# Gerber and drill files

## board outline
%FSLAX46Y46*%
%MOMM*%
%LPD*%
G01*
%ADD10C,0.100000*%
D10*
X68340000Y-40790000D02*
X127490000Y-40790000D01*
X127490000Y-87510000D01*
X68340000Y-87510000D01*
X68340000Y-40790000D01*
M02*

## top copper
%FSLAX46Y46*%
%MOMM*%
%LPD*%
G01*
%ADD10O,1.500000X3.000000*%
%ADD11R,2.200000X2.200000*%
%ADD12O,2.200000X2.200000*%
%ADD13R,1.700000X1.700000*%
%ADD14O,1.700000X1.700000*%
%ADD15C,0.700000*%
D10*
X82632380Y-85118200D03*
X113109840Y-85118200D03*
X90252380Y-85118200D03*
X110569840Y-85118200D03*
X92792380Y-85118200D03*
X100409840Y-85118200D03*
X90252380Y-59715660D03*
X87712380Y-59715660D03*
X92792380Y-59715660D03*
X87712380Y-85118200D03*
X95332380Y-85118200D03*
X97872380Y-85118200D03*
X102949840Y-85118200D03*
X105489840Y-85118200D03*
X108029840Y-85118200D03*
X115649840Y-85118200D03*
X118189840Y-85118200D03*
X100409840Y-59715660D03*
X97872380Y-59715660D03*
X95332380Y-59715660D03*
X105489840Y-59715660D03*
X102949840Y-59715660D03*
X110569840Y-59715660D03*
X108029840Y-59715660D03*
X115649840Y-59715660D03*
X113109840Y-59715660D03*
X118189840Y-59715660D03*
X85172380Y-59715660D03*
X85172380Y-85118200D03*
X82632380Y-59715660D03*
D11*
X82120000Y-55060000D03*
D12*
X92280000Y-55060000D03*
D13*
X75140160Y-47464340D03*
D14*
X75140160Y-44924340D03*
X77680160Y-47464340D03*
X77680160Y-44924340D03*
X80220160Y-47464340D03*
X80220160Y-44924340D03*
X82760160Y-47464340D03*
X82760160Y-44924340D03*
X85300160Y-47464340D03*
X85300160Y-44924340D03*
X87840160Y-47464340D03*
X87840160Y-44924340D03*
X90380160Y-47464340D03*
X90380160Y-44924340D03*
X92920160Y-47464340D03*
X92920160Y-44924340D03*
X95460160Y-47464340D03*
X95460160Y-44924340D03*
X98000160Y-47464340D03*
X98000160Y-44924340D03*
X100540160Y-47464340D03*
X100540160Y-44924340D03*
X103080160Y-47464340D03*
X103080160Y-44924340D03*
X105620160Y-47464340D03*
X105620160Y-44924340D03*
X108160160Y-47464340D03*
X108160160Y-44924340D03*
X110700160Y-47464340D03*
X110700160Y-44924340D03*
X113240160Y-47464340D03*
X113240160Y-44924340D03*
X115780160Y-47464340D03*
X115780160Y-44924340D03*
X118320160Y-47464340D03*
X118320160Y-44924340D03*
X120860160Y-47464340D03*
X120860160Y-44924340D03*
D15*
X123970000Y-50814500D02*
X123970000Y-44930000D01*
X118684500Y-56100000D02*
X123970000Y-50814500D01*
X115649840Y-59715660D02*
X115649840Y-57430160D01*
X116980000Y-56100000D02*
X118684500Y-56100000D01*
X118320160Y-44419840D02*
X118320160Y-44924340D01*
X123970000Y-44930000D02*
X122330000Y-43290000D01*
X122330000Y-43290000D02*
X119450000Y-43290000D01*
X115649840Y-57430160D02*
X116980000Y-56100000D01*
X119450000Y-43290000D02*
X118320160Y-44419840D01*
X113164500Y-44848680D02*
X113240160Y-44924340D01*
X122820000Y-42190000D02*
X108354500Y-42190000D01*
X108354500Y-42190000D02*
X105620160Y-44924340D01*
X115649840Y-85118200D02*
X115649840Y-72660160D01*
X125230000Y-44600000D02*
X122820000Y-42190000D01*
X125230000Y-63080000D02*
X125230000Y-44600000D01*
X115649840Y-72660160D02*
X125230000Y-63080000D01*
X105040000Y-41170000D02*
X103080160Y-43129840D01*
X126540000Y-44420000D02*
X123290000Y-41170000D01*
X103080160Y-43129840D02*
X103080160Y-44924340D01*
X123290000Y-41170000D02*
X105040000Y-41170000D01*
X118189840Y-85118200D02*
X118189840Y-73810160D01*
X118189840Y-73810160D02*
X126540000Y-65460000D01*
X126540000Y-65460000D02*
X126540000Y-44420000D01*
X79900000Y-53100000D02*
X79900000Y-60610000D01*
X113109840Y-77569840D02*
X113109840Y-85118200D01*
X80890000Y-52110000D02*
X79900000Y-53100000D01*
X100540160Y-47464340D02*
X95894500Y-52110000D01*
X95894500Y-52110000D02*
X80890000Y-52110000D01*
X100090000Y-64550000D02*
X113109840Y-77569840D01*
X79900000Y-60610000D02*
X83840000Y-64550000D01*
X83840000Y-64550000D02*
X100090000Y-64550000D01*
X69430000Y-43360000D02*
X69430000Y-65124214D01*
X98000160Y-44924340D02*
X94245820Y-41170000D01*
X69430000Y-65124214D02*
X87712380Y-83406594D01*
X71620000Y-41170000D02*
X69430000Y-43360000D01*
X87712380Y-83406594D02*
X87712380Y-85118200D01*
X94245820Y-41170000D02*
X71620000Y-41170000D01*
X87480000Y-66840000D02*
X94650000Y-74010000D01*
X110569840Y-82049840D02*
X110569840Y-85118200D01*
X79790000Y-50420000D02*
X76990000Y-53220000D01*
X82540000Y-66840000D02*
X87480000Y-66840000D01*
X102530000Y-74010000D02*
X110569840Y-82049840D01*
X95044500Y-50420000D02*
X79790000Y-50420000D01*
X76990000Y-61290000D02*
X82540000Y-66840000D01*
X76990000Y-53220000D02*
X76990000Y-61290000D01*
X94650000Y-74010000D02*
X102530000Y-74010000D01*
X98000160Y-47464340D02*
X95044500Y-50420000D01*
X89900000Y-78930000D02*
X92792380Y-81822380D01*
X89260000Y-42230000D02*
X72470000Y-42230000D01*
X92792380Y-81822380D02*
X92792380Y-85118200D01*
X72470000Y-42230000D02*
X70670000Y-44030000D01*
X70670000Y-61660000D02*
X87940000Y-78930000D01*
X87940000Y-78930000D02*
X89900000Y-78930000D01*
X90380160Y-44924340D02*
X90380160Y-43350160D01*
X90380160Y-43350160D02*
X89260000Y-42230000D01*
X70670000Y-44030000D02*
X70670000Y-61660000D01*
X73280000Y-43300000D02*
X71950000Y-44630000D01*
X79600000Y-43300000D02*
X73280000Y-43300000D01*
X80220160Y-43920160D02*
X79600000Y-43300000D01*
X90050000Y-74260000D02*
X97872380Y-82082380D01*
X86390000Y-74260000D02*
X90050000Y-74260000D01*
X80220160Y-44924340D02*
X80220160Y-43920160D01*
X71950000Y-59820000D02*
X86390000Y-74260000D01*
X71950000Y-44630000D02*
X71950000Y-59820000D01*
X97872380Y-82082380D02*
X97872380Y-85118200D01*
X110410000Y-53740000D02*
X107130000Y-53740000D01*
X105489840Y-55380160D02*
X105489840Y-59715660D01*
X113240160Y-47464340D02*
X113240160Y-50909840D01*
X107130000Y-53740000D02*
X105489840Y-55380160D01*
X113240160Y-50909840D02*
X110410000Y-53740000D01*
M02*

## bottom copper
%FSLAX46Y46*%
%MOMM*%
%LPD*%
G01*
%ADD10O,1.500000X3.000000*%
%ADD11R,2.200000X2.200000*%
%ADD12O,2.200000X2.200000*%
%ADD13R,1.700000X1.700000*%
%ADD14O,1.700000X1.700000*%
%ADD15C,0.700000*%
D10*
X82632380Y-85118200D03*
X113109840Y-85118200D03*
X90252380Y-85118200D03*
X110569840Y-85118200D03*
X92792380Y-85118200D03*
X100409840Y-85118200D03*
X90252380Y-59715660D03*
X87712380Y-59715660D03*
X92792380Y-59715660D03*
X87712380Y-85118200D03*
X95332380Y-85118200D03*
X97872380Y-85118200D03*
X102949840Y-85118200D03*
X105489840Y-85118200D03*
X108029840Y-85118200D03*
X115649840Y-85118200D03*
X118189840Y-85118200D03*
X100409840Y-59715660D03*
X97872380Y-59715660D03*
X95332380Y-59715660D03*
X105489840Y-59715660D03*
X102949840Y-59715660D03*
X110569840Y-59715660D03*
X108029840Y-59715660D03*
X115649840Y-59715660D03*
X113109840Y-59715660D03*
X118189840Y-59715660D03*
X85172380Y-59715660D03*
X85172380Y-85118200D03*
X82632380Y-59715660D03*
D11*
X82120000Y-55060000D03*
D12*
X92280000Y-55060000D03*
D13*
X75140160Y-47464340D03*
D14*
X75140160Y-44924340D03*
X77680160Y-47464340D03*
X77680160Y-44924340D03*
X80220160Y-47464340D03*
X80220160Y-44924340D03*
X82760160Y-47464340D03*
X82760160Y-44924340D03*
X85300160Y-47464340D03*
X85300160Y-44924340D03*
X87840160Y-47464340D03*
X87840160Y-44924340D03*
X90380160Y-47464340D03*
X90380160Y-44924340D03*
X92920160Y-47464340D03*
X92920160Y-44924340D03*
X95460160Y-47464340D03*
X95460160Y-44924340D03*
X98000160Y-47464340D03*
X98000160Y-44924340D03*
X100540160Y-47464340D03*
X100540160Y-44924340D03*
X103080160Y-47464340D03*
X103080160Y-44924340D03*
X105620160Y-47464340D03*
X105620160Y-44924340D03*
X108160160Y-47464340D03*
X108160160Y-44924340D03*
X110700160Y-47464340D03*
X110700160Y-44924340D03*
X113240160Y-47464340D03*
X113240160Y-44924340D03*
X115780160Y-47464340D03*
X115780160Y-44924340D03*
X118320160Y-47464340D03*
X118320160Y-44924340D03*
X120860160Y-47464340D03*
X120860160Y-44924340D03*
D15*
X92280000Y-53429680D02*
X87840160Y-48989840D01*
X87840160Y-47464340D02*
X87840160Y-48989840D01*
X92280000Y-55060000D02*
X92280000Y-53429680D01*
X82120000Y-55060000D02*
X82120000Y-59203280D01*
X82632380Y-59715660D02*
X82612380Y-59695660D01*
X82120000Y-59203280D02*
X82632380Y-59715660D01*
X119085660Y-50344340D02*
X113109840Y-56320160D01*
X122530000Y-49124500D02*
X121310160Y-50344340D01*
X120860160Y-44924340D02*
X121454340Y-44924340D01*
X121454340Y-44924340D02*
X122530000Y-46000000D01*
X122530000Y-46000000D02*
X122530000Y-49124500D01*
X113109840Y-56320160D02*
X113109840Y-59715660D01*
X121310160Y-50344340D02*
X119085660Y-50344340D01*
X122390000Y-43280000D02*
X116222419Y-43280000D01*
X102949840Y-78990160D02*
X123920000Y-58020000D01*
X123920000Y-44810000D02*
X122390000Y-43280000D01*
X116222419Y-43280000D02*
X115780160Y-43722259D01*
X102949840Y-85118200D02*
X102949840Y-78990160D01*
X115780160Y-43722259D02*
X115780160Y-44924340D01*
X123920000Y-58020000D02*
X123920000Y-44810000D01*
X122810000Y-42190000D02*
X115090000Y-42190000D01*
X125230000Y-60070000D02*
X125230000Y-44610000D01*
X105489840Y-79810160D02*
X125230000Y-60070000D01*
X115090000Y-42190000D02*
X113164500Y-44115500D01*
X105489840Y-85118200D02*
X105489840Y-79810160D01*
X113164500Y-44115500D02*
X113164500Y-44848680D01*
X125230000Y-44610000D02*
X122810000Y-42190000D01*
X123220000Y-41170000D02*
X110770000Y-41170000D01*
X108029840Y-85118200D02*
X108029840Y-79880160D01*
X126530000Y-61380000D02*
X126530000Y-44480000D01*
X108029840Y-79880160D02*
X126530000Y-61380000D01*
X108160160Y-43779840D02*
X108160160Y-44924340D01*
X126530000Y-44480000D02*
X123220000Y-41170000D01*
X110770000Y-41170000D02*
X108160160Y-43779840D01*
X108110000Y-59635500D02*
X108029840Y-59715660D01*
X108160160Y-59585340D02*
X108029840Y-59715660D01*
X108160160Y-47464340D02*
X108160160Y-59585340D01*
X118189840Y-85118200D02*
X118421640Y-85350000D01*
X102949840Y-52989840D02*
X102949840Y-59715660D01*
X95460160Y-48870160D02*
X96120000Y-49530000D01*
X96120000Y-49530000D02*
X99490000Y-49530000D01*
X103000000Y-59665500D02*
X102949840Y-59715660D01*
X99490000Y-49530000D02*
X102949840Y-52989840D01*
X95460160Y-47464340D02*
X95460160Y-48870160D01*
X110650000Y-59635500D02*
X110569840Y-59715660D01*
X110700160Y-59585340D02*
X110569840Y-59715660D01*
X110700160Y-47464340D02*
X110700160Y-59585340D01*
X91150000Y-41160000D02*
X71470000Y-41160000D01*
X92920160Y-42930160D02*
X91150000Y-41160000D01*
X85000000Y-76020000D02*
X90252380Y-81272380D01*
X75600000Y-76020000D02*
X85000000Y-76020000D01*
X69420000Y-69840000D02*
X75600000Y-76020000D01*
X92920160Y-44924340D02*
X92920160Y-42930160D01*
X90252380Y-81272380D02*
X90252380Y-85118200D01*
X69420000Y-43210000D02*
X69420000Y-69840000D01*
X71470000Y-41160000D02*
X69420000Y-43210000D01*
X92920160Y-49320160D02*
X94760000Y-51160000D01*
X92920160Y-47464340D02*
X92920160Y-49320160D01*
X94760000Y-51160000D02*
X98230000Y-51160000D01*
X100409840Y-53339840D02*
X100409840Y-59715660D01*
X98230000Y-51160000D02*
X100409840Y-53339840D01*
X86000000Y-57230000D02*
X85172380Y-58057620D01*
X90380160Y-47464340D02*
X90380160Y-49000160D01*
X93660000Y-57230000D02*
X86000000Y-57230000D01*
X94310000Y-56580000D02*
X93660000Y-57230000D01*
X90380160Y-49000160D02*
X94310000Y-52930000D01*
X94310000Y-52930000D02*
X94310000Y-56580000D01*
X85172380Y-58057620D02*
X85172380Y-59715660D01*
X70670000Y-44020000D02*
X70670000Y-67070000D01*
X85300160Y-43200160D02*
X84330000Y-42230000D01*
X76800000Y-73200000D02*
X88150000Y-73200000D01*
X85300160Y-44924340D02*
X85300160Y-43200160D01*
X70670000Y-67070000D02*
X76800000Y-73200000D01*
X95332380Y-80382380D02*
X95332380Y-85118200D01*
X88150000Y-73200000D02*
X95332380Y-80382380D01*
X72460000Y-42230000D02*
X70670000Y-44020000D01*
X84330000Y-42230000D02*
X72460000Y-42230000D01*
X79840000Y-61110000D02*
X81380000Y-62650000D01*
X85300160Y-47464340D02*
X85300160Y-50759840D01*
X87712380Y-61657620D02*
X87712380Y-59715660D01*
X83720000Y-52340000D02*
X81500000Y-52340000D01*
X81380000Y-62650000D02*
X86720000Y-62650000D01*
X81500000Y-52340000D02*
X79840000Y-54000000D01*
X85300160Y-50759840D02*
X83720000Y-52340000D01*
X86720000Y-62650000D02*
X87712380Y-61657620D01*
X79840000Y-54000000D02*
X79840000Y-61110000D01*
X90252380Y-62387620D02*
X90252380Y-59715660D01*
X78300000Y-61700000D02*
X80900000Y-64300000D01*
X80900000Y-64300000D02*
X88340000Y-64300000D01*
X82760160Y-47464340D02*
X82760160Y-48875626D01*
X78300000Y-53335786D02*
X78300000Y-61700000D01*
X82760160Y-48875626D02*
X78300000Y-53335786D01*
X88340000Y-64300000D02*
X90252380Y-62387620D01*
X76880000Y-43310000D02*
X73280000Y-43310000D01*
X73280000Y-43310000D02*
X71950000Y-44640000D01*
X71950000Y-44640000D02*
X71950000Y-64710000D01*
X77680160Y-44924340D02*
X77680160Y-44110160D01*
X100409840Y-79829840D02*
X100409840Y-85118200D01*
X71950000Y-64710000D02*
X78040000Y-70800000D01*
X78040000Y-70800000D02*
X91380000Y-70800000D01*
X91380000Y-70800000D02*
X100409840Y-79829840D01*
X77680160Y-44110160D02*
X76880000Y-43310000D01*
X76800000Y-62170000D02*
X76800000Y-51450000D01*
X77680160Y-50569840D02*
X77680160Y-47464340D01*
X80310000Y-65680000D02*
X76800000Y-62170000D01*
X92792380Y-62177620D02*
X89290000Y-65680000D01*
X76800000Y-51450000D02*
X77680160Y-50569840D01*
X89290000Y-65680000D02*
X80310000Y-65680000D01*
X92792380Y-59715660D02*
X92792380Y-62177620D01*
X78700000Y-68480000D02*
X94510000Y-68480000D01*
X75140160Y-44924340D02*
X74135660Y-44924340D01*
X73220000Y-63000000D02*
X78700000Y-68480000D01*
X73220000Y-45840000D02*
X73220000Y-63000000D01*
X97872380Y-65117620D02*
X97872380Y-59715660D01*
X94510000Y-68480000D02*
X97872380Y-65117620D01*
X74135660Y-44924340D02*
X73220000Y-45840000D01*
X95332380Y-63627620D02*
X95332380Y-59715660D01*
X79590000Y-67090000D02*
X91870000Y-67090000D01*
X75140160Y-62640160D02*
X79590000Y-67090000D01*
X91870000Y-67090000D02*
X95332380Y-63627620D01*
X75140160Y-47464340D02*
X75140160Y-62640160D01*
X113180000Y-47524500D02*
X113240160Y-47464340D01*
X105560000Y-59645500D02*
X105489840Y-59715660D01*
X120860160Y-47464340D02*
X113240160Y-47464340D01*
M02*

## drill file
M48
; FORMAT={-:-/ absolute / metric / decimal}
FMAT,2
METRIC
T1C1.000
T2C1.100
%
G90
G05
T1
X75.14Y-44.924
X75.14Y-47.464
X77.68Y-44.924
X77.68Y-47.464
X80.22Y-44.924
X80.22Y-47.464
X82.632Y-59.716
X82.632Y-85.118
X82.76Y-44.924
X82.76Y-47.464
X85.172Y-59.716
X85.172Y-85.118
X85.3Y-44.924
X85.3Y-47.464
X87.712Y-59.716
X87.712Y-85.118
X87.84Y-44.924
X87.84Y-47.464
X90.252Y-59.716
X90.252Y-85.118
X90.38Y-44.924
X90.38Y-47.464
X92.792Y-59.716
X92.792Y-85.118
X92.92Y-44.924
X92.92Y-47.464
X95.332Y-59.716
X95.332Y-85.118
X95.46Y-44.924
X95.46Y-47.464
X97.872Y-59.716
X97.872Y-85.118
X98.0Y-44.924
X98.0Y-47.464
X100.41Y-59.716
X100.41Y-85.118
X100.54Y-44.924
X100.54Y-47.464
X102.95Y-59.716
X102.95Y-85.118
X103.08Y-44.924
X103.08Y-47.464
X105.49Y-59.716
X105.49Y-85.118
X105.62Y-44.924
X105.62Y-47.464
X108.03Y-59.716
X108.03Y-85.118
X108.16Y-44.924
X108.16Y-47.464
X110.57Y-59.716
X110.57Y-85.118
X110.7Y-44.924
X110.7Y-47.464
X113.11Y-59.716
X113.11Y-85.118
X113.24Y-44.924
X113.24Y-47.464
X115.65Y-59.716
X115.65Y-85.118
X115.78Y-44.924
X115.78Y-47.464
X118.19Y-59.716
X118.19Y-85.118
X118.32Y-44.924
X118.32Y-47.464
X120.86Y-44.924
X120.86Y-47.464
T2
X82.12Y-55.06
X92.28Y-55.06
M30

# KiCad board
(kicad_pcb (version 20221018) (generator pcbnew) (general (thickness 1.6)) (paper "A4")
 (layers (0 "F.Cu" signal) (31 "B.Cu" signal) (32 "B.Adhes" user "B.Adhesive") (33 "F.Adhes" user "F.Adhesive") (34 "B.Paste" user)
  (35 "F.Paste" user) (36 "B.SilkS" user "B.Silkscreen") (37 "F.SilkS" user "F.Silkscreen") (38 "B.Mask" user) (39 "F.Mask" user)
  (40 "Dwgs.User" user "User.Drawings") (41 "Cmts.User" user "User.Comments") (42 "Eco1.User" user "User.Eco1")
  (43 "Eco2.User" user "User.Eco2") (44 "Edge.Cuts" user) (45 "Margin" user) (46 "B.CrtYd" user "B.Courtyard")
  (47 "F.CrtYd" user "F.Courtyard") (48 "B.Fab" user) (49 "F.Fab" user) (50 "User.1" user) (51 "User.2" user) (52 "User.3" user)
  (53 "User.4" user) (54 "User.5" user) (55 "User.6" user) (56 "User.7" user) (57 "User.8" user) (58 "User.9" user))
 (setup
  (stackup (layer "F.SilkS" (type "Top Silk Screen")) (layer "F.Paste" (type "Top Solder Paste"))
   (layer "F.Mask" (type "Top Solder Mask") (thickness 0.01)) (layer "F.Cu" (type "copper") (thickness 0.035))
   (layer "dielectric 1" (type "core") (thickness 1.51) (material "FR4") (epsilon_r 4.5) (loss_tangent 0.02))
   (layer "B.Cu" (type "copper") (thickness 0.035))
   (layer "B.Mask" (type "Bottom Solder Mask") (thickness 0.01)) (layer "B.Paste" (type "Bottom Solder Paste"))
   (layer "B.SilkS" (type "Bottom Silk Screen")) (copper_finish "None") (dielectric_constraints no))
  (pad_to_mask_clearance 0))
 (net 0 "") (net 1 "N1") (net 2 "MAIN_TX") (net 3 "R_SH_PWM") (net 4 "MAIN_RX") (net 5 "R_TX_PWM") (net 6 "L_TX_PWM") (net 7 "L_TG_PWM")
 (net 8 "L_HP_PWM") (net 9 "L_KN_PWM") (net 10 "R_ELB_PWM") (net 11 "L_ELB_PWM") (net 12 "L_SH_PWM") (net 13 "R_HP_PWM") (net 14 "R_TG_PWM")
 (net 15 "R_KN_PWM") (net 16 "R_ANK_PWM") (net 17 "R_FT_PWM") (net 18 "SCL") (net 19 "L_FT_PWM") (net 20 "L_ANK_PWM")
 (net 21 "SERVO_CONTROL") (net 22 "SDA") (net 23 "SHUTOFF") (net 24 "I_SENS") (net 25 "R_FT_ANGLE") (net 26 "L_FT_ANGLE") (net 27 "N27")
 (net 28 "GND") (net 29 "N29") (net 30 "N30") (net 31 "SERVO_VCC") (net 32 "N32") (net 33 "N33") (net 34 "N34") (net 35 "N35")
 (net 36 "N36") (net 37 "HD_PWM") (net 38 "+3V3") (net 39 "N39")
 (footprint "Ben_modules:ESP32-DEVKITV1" (layer "F.Cu") (at 99.15 72.85)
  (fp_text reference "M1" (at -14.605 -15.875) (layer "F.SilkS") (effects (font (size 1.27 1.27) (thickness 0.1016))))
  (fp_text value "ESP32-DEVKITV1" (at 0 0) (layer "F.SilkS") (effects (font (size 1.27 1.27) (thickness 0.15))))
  (pad "3V3" thru_hole oval (at -16.51762 12.2682) (size 1.5 3) (drill 1) (layers "*.Cu" "*.Mask") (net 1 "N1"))
  (pad "D1" thru_hole oval (at 13.95984 12.2682) (size 1.5 3) (drill 1) (layers "*.Cu" "*.Mask") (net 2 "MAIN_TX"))
  (pad "D2" thru_hole oval (at -8.89762 12.2682) (size 1.5 3) (drill 1) (layers "*.Cu" "*.Mask") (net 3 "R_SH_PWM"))
  (pad "D3" thru_hole oval (at 11.41984 12.2682) (size 1.5 3) (drill 1) (layers "*.Cu" "*.Mask") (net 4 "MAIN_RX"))
  (pad "D4" thru_hole oval (at -6.35762 12.2682) (size 1.5 3) (drill 1) (layers "*.Cu" "*.Mask") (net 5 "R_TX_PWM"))
  (pad "D5" thru_hole oval (at 1.25984 12.2682) (size 1.5 3) (drill 1) (layers "*.Cu" "*.Mask") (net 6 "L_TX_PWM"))
  (pad "D12" thru_hole oval (at -8.89762 -13.13434) (size 1.5 3) (drill 1) (layers "*.Cu" "*.Mask") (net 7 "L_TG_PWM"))
  (pad "D13" thru_hole oval (at -11.43762 -13.13434) (size 1.5 3) (drill 1) (layers "*.Cu" "*.Mask") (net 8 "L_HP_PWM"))
  (pad "D14" thru_hole oval (at -6.35762 -13.13434) (size 1.5 3) (drill 1) (layers "*.Cu" "*.Mask") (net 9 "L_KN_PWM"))
  (pad "D15" thru_hole oval (at -11.43762 12.2682) (size 1.5 3) (drill 1) (layers "*.Cu" "*.Mask") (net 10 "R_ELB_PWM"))
  (pad "D16" thru_hole oval (at -3.81762 12.2682) (size 1.5 3) (drill 1) (layers "*.Cu" "*.Mask") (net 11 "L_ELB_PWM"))
  (pad "D17" thru_hole oval (at -1.27762 12.2682) (size 1.5 3) (drill 1) (layers "*.Cu" "*.Mask") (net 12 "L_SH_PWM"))
  (pad "D18" thru_hole oval (at 3.79984 12.2682) (size 1.5 3) (drill 1) (layers "*.Cu" "*.Mask") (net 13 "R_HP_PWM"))
  (pad "D19" thru_hole oval (at 6.33984 12.2682) (size 1.5 3) (drill 1) (layers "*.Cu" "*.Mask") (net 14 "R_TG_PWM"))
  (pad "D21" thru_hole oval (at 8.87984 12.2682) (size 1.5 3) (drill 1) (layers "*.Cu" "*.Mask") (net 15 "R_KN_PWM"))
  (pad "D22" thru_hole oval (at 16.49984 12.2682) (size 1.5 3) (drill 1) (layers "*.Cu" "*.Mask") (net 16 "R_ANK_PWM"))
  (pad "D23" thru_hole oval (at 19.03984 12.2682) (size 1.5 3) (drill 1) (layers "*.Cu" "*.Mask") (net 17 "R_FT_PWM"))
  (pad "D25" thru_hole oval (at 1.25984 -13.13434) (size 1.5 3) (drill 1) (layers "*.Cu" "*.Mask") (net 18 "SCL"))
  (pad "D26" thru_hole oval (at -1.27762 -13.13434) (size 1.5 3) (drill 1) (layers "*.Cu" "*.Mask") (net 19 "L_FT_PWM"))
  (pad "D27" thru_hole oval (at -3.81762 -13.13434) (size 1.5 3) (drill 1) (layers "*.Cu" "*.Mask") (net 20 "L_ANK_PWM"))
  (pad "D32" thru_hole oval (at 6.33984 -13.13434) (size 1.5 3) (drill 1) (layers "*.Cu" "*.Mask") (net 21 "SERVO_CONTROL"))
  (pad "D33" thru_hole oval (at 3.79984 -13.13434) (size 1.5 3) (drill 1) (layers "*.Cu" "*.Mask") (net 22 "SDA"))
  (pad "D34" thru_hole oval (at 11.41984 -13.13434) (size 1.5 3) (drill 1) (layers "*.Cu" "*.Mask") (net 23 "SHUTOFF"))
  (pad "D35" thru_hole oval (at 8.87984 -13.13434) (size 1.5 3) (drill 1) (layers "*.Cu" "*.Mask") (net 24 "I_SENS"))
  (pad "D36" thru_hole oval (at 16.49984 -13.13434) (size 1.5 3) (drill 1) (layers "*.Cu" "*.Mask") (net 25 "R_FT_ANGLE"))
  (pad "D39" thru_hole oval (at 13.95984 -13.13434) (size 1.5 3) (drill 1) (layers "*.Cu" "*.Mask") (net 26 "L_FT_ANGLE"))
  (pad "EN" thru_hole oval (at 19.03984 -13.13434) (size 1.5 3) (drill 1) (layers "*.Cu" "*.Mask") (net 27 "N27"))
  (pad "GND@1" thru_hole oval (at -13.97762 -13.13434) (size 1.5 3) (drill 1) (layers "*.Cu" "*.Mask") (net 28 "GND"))
  (pad "GND@2" thru_hole oval (at -13.97762 12.2682) (size 1.5 3) (drill 1) (layers "*.Cu" "*.Mask") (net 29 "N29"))
  (pad "VIN" thru_hole oval (at -16.51762 -13.13434) (size 1.5 3) (drill 1) (layers "*.Cu" "*.Mask") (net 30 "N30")))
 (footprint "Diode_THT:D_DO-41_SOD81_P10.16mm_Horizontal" (layer "F.Cu") (at 82.12 55.06)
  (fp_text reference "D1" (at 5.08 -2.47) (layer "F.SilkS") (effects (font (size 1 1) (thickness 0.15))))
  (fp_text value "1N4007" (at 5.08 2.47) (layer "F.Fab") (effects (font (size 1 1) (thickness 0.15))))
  (pad "1" thru_hole rect (at 0 0) (size 2.2 2.2) (drill 1.1) (layers "*.Cu" "*.Mask") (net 30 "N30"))
  (pad "2" thru_hole oval (at 10.16 0) (size 2.2 2.2) (drill 1.1) (layers "*.Cu" "*.Mask") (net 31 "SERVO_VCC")))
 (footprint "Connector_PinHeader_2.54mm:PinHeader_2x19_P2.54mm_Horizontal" (layer "F.Cu") (at 75.14016 47.46434 90)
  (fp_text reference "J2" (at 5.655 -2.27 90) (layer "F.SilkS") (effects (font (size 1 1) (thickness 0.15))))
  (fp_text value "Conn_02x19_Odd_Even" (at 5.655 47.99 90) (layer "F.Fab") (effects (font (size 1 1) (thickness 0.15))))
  (pad "1" thru_hole rect (at 0 0 90) (size 1.7 1.7) (drill 1) (layers "*.Cu" "*.Mask") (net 20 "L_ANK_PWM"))
  (pad "2" thru_hole oval (at 2.54 0 90) (size 1.7 1.7) (drill 1) (layers "*.Cu" "*.Mask") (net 19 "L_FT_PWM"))
  (pad "3" thru_hole oval (at 0 2.54 90) (size 1.7 1.7) (drill 1) (layers "*.Cu" "*.Mask") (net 9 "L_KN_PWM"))
  (pad "4" thru_hole oval (at 2.54 2.54 90) (size 1.7 1.7) (drill 1) (layers "*.Cu" "*.Mask") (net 6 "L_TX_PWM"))
  (pad "5" thru_hole oval (at 0 5.08 90) (size 1.7 1.7) (drill 1) (layers "*.Cu" "*.Mask") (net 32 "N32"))
  (pad "6" thru_hole oval (at 2.54 5.08 90) (size 1.7 1.7) (drill 1) (layers "*.Cu" "*.Mask") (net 12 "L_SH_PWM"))
  (pad "7" thru_hole oval (at 0 7.62 90) (size 1.7 1.7) (drill 1) (layers "*.Cu" "*.Mask") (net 7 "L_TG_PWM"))
  (pad "8" thru_hole oval (at 2.54 7.62 90) (size 1.7 1.7) (drill 1) (layers "*.Cu" "*.Mask") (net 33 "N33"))
  (pad "9" thru_hole oval (at 0 10.16 90) (size 1.7 1.7) (drill 1) (layers "*.Cu" "*.Mask") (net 8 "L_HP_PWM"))
  (pad "10" thru_hole oval (at 2.54 10.16 90) (size 1.7 1.7) (drill 1) (layers "*.Cu" "*.Mask") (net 11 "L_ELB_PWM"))
  (pad "11" thru_hole oval (at 0 12.7 90) (size 1.7 1.7) (drill 1) (layers "*.Cu" "*.Mask") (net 31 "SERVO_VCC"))
  (pad "12" thru_hole oval (at 2.54 12.7 90) (size 1.7 1.7) (drill 1) (layers "*.Cu" "*.Mask") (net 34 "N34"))
  (pad "13" thru_hole oval (at 0 15.24 90) (size 1.7 1.7) (drill 1) (layers "*.Cu" "*.Mask") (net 28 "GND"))
  (pad "14" thru_hole oval (at 2.54 15.24 90) (size 1.7 1.7) (drill 1) (layers "*.Cu" "*.Mask") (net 5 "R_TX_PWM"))
  (pad "15" thru_hole oval (at 0 17.78 90) (size 1.7 1.7) (drill 1) (layers "*.Cu" "*.Mask") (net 18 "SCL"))
  (pad "16" thru_hole oval (at 2.54 17.78 90) (size 1.7 1.7) (drill 1) (layers "*.Cu" "*.Mask") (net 3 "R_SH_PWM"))
  (pad "17" thru_hole oval (at 0 20.32 90) (size 1.7 1.7) (drill 1) (layers "*.Cu" "*.Mask") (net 22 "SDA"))
  (pad "18" thru_hole oval (at 2.54 20.32 90) (size 1.7 1.7) (drill 1) (layers "*.Cu" "*.Mask") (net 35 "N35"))
  (pad "19" thru_hole oval (at 0 22.86 90) (size 1.7 1.7) (drill 1) (layers "*.Cu" "*.Mask") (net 4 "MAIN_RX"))
  (pad "20" thru_hole oval (at 2.54 22.86 90) (size 1.7 1.7) (drill 1) (layers "*.Cu" "*.Mask") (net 10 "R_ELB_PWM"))
  (pad "21" thru_hole oval (at 0 25.4 90) (size 1.7 1.7) (drill 1) (layers "*.Cu" "*.Mask") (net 2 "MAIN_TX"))
  (pad "22" thru_hole oval (at 2.54 25.4 90) (size 1.7 1.7) (drill 1) (layers "*.Cu" "*.Mask") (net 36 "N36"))
  (pad "23" thru_hole oval (at 0 27.94 90) (size 1.7 1.7) (drill 1) (layers "*.Cu" "*.Mask") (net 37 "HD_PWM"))
  (pad "24" thru_hole oval (at 2.54 27.94 90) (size 1.7 1.7) (drill 1) (layers "*.Cu" "*.Mask") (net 17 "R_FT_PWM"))
  (pad "25" thru_hole oval (at 0 30.48 90) (size 1.7 1.7) (drill 1) (layers "*.Cu" "*.Mask") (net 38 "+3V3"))
  (pad "26" thru_hole oval (at 2.54 30.48 90) (size 1.7 1.7) (drill 1) (layers "*.Cu" "*.Mask") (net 16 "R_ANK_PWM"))
  (pad "27" thru_hole oval (at 0 33.02 90) (size 1.7 1.7) (drill 1) (layers "*.Cu" "*.Mask") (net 24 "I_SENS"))
  (pad "28" thru_hole oval (at 2.54 33.02 90) (size 1.7 1.7) (drill 1) (layers "*.Cu" "*.Mask") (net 15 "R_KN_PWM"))
  (pad "29" thru_hole oval (at 0 35.56 90) (size 1.7 1.7) (drill 1) (layers "*.Cu" "*.Mask") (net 23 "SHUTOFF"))
  (pad "30" thru_hole oval (at 2.54 35.56 90) (size 1.7 1.7) (drill 1) (layers "*.Cu" "*.Mask") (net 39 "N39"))
  (pad "31" thru_hole oval (at 0 38.1 90) (size 1.7 1.7) (drill 1) (layers "*.Cu" "*.Mask") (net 21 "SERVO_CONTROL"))
  (pad "32" thru_hole oval (at 2.54 38.1 90) (size 1.7 1.7) (drill 1) (layers "*.Cu" "*.Mask") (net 14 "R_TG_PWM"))
  (pad "33" thru_hole oval (at 0 40.64 90) (size 1.7 1.7) (drill 1) (layers "*.Cu" "*.Mask") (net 21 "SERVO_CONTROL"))
  (pad "34" thru_hole oval (at 2.54 40.64 90) (size 1.7 1.7) (drill 1) (layers "*.Cu" "*.Mask") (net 13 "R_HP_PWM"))
  (pad "35" thru_hole oval (at 0 43.18 90) (size 1.7 1.7) (drill 1) (layers "*.Cu" "*.Mask") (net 21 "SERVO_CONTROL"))
  (pad "36" thru_hole oval (at 2.54 43.18 90) (size 1.7 1.7) (drill 1) (layers "*.Cu" "*.Mask") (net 25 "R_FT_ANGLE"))
  (pad "37" thru_hole oval (at 0 45.72 90) (size 1.7 1.7) (drill 1) (layers "*.Cu" "*.Mask") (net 21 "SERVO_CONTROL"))
  (pad "38" thru_hole oval (at 2.54 45.72 90) (size 1.7 1.7) (drill 1) (layers "*.Cu" "*.Mask") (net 26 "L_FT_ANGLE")))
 (gr_rect (start 68.34 40.79) (end 127.49 87.51) (stroke (width 0.1) (type default)) (fill none) (layer "Edge.Cuts"))
 (segment (start 92.28 53.42968) (end 87.84016 48.98984) (width 0.7) (layer "B.Cu") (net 31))
 (segment (start 87.84016 47.46434) (end 87.84016 48.98984) (width 0.7) (layer "B.Cu") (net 31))
 (segment (start 92.28 55.06) (end 92.28 53.42968) (width 0.7) (layer "B.Cu") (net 31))
 (segment (start 82.12 55.06) (end 82.12 59.20328) (width 0.7) (layer "B.Cu") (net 30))
 (segment (start 82.63238 59.71566) (end 82.61238 59.69566) (width 0.7) (layer "B.Cu") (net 30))
 (segment (start 82.12 59.20328) (end 82.63238 59.71566) (width 0.7) (layer "B.Cu") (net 30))
 (segment (start 119.08566 50.34434) (end 113.10984 56.32016) (width 0.7) (layer "B.Cu") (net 26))
 (segment (start 122.53 49.1245) (end 121.31016 50.34434) (width 0.7) (layer "B.Cu") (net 26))
 (segment (start 120.86016 44.92434) (end 121.45434 44.92434) (width 0.7) (layer "B.Cu") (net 26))
 (segment (start 121.45434 44.92434) (end 122.53 46) (width 0.7) (layer "B.Cu") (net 26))
 (segment (start 122.53 46) (end 122.53 49.1245) (width 0.7) (layer "B.Cu") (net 26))
 (segment (start 113.10984 56.32016) (end 113.10984 59.71566) (width 0.7) (layer "B.Cu") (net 26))
 (segment (start 121.31016 50.34434) (end 119.08566 50.34434) (width 0.7) (layer "B.Cu") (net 26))
 (segment (start 123.97 50.8145) (end 123.97 44.93) (width 0.7) (layer "F.Cu") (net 25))
 (segment (start 118.6845 56.1) (end 123.97 50.8145) (width 0.7) (layer "F.Cu") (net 25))
 (segment (start 115.64984 59.71566) (end 115.64984 57.43016) (width 0.7) (layer "F.Cu") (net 25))
 (segment (start 116.98 56.1) (end 118.6845 56.1) (width 0.7) (layer "F.Cu") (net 25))
 (segment (start 118.32016 44.41984) (end 118.32016 44.92434) (width 0.7) (layer "F.Cu") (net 25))
 (segment (start 123.97 44.93) (end 122.33 43.29) (width 0.7) (layer "F.Cu") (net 25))
 (segment (start 122.33 43.29) (end 119.45 43.29) (width 0.7) (layer "F.Cu") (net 25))
 (segment (start 115.64984 57.43016) (end 116.98 56.1) (width 0.7) (layer "F.Cu") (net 25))
 (segment (start 119.45 43.29) (end 118.32016 44.41984) (width 0.7) (layer "F.Cu") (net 25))
 (segment (start 122.39 43.28) (end 116.222419 43.28) (width 0.7) (layer "B.Cu") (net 13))
 (segment (start 102.94984 78.99016) (end 123.92 58.02) (width 0.7) (layer "B.Cu") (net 13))
 (segment (start 123.92 44.81) (end 122.39 43.28) (width 0.7) (layer "B.Cu") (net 13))
 (segment (start 116.222419 43.28) (end 115.78016 43.722259) (width 0.7) (layer "B.Cu") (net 13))
 (segment (start 102.94984 85.1182) (end 102.94984 78.99016) (width 0.7) (layer "B.Cu") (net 13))
 (segment (start 115.78016 43.722259) (end 115.78016 44.92434) (width 0.7) (layer "B.Cu") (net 13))
 (segment (start 123.92 58.02) (end 123.92 44.81) (width 0.7) (layer "B.Cu") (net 13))
 (segment (start 113.1645 44.84868) (end 113.24016 44.92434) (width 0.7) (layer "F.Cu") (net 14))
 (segment (start 122.81 42.19) (end 115.09 42.19) (width 0.7) (layer "B.Cu") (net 14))
 (segment (start 125.23 60.07) (end 125.23 44.61) (width 0.7) (layer "B.Cu") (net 14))
 (segment (start 105.48984 79.81016) (end 125.23 60.07) (width 0.7) (layer "B.Cu") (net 14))
 (segment (start 115.09 42.19) (end 113.1645 44.1155) (width 0.7) (layer "B.Cu") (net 14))
 (segment (start 105.48984 85.1182) (end 105.48984 79.81016) (width 0.7) (layer "B.Cu") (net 14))
 (segment (start 113.1645 44.1155) (end 113.1645 44.84868) (width 0.7) (layer "B.Cu") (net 14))
 (segment (start 125.23 44.61) (end 122.81 42.19) (width 0.7) (layer "B.Cu") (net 14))
 (segment (start 123.22 41.17) (end 110.77 41.17) (width 0.7) (layer "B.Cu") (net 15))
 (segment (start 108.02984 85.1182) (end 108.02984 79.88016) (width 0.7) (layer "B.Cu") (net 15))
 (segment (start 126.53 61.38) (end 126.53 44.48) (width 0.7) (layer "B.Cu") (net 15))
 (segment (start 108.02984 79.88016) (end 126.53 61.38) (width 0.7) (layer "B.Cu") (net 15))
 (segment (start 108.16016 43.77984) (end 108.16016 44.92434) (width 0.7) (layer "B.Cu") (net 15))
 (segment (start 126.53 44.48) (end 123.22 41.17) (width 0.7) (layer "B.Cu") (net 15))
 (segment (start 110.77 41.17) (end 108.16016 43.77984) (width 0.7) (layer "B.Cu") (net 15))
 (segment (start 108.11 59.6355) (end 108.02984 59.71566) (width 0.7) (layer "B.Cu") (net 24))
 (segment (start 108.16016 59.58534) (end 108.02984 59.71566) (width 0.7) (layer "B.Cu") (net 24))
 (segment (start 108.16016 47.46434) (end 108.16016 59.58534) (width 0.7) (layer "B.Cu") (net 24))
 (segment (start 122.82 42.19) (end 108.3545 42.19) (width 0.7) (layer "F.Cu") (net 16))
 (segment (start 108.3545 42.19) (end 105.62016 44.92434) (width 0.7) (layer "F.Cu") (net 16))
 (segment (start 115.64984 85.1182) (end 115.64984 72.66016) (width 0.7) (layer "F.Cu") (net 16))
 (segment (start 125.23 44.6) (end 122.82 42.19) (width 0.7) (layer "F.Cu") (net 16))
 (segment (start 125.23 63.08) (end 125.23 44.6) (width 0.7) (layer "F.Cu") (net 16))
 (segment (start 115.64984 72.66016) (end 125.23 63.08) (width 0.7) (layer "F.Cu") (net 16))
 (segment (start 105.04 41.17) (end 103.08016 43.12984) (width 0.7) (layer "F.Cu") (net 17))
 (segment (start 126.54 44.42) (end 123.29 41.17) (width 0.7) (layer "F.Cu") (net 17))
 (segment (start 103.08016 43.12984) (end 103.08016 44.92434) (width 0.7) (layer "F.Cu") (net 17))
 (segment (start 123.29 41.17) (end 105.04 41.17) (width 0.7) (layer "F.Cu") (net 17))
 (segment (start 118.18984 85.1182) (end 118.18984 73.81016) (width 0.7) (layer "F.Cu") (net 17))
 (segment (start 118.18984 73.81016) (end 126.54 65.46) (width 0.7) (layer "F.Cu") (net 17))
 (segment (start 126.54 65.46) (end 126.54 44.42) (width 0.7) (layer "F.Cu") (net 17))
 (segment (start 118.18984 85.1182) (end 118.42164 85.35) (width 0.7) (layer "B.Cu") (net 17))
 (segment (start 79.9 53.1) (end 79.9 60.61) (width 0.7) (layer "F.Cu") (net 2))
 (segment (start 113.10984 77.56984) (end 113.10984 85.1182) (width 0.7) (layer "F.Cu") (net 2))
 (segment (start 80.89 52.11) (end 79.9 53.1) (width 0.7) (layer "F.Cu") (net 2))
 (segment (start 100.54016 47.46434) (end 95.8945 52.11) (width 0.7) (layer "F.Cu") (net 2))
 (segment (start 95.8945 52.11) (end 80.89 52.11) (width 0.7) (layer "F.Cu") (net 2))
 (segment (start 100.09 64.55) (end 113.10984 77.56984) (width 0.7) (layer "F.Cu") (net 2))
 (segment (start 79.9 60.61) (end 83.84 64.55) (width 0.7) (layer "F.Cu") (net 2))
 (segment (start 83.84 64.55) (end 100.09 64.55) (width 0.7) (layer "F.Cu") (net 2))
 (segment (start 69.43 43.36) (end 69.43 65.124214) (width 0.7) (layer "F.Cu") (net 10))
 (segment (start 98.00016 44.92434) (end 94.24582 41.17) (width 0.7) (layer "F.Cu") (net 10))
 (segment (start 69.43 65.124214) (end 87.71238 83.406594) (width 0.7) (layer "F.Cu") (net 10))
 (segment (start 71.62 41.17) (end 69.43 43.36) (width 0.7) (layer "F.Cu") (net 10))
 (segment (start 87.71238 83.406594) (end 87.71238 85.1182) (width 0.7) (layer "F.Cu") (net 10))
 (segment (start 94.24582 41.17) (end 71.62 41.17) (width 0.7) (layer "F.Cu") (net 10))
 (segment (start 87.48 66.84) (end 94.65 74.01) (width 0.7) (layer "F.Cu") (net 4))
 (segment (start 110.56984 82.04984) (end 110.56984 85.1182) (width 0.7) (layer "F.Cu") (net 4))
 (segment (start 79.79 50.42) (end 76.99 53.22) (width 0.7) (layer "F.Cu") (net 4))
 (segment (start 82.54 66.84) (end 87.48 66.84) (width 0.7) (layer "F.Cu") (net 4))
 (segment (start 102.53 74.01) (end 110.56984 82.04984) (width 0.7) (layer "F.Cu") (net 4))
 (segment (start 95.0445 50.42) (end 79.79 50.42) (width 0.7) (layer "F.Cu") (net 4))
 (segment (start 76.99 61.29) (end 82.54 66.84) (width 0.7) (layer "F.Cu") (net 4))
 (segment (start 76.99 53.22) (end 76.99 61.29) (width 0.7) (layer "F.Cu") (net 4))
 (segment (start 94.65 74.01) (end 102.53 74.01) (width 0.7) (layer "F.Cu") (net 4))
 (segment (start 98.00016 47.46434) (end 95.0445 50.42) (width 0.7) (layer "F.Cu") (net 4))
 (segment (start 102.94984 52.98984) (end 102.94984 59.71566) (width 0.7) (layer "B.Cu") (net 22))
 (segment (start 95.46016 48.87016) (end 96.12 49.53) (width 0.7) (layer "B.Cu") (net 22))
 (segment (start 96.12 49.53) (end 99.49 49.53) (width 0.7) (layer "B.Cu") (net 22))
 (segment (start 103 59.6655) (end 102.94984 59.71566) (width 0.7) (layer "B.Cu") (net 22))
 (segment (start 99.49 49.53) (end 102.94984 52.98984) (width 0.7) (layer "B.Cu") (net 22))
 (segment (start 95.46016 47.46434) (end 95.46016 48.87016) (width 0.7) (layer "B.Cu") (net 22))
 (segment (start 110.65 59.6355) (end 110.56984 59.71566) (width 0.7) (layer "B.Cu") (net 23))
 (segment (start 110.70016 59.58534) (end 110.56984 59.71566) (width 0.7) (layer "B.Cu") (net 23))
 (segment (start 110.70016 47.46434) (end 110.70016 59.58534) (width 0.7) (layer "B.Cu") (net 23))
 (segment (start 91.15 41.16) (end 71.47 41.16) (width 0.7) (layer "B.Cu") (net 3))
 (segment (start 92.92016 42.93016) (end 91.15 41.16) (width 0.7) (layer "B.Cu") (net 3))
 (segment (start 85 76.02) (end 90.25238 81.27238) (width 0.7) (layer "B.Cu") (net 3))
 (segment (start 75.6 76.02) (end 85 76.02) (width 0.7) (layer "B.Cu") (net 3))
 (segment (start 69.42 69.84) (end 75.6 76.02) (width 0.7) (layer "B.Cu") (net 3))
 (segment (start 92.92016 44.92434) (end 92.92016 42.93016) (width 0.7) (layer "B.Cu") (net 3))
 (segment (start 90.25238 81.27238) (end 90.25238 85.1182) (width 0.7) (layer "B.Cu") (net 3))
 (segment (start 69.42 43.21) (end 69.42 69.84) (width 0.7) (layer "B.Cu") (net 3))
 (segment (start 71.47 41.16) (end 69.42 43.21) (width 0.7) (layer "B.Cu") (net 3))
 (segment (start 92.92016 49.32016) (end 94.76 51.16) (width 0.7) (layer "B.Cu") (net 18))
 (segment (start 92.92016 47.46434) (end 92.92016 49.32016) (width 0.7) (layer "B.Cu") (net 18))
 (segment (start 94.76 51.16) (end 98.23 51.16) (width 0.7) (layer "B.Cu") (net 18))
 (segment (start 100.40984 53.33984) (end 100.40984 59.71566) (width 0.7) (layer "B.Cu") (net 18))
 (segment (start 98.23 51.16) (end 100.40984 53.33984) (width 0.7) (layer "B.Cu") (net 18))
 (segment (start 89.9 78.93) (end 92.79238 81.82238) (width 0.7) (layer "F.Cu") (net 5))
 (segment (start 89.26 42.23) (end 72.47 42.23) (width 0.7) (layer "F.Cu") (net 5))
 (segment (start 92.79238 81.82238) (end 92.79238 85.1182) (width 0.7) (layer "F.Cu") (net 5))
 (segment (start 72.47 42.23) (end 70.67 44.03) (width 0.7) (layer "F.Cu") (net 5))
 (segment (start 70.67 61.66) (end 87.94 78.93) (width 0.7) (layer "F.Cu") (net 5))
 (segment (start 87.94 78.93) (end 89.9 78.93) (width 0.7) (layer "F.Cu") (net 5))
 (segment (start 90.38016 44.92434) (end 90.38016 43.35016) (width 0.7) (layer "F.Cu") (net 5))
 (segment (start 90.38016 43.35016) (end 89.26 42.23) (width 0.7) (layer "F.Cu") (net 5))
 (segment (start 70.67 44.03) (end 70.67 61.66) (width 0.7) (layer "F.Cu") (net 5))
 (segment (start 86 57.23) (end 85.17238 58.05762) (width 0.7) (layer "B.Cu") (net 28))
 (segment (start 90.38016 47.46434) (end 90.38016 49.00016) (width 0.7) (layer "B.Cu") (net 28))
 (segment (start 93.66 57.23) (end 86 57.23) (width 0.7) (layer "B.Cu") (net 28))
 (segment (start 94.31 56.58) (end 93.66 57.23) (width 0.7) (layer "B.Cu") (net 28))
 (segment (start 90.38016 49.00016) (end 94.31 52.93) (width 0.7) (layer "B.Cu") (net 28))
 (segment (start 94.31 52.93) (end 94.31 56.58) (width 0.7) (layer "B.Cu") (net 28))
 (segment (start 85.17238 58.05762) (end 85.17238 59.71566) (width 0.7) (layer "B.Cu") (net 28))
 (segment (start 70.67 44.02) (end 70.67 67.07) (width 0.7) (layer "B.Cu") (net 11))
 (segment (start 85.30016 43.20016) (end 84.33 42.23) (width 0.7) (layer "B.Cu") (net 11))
 (segment (start 76.8 73.2) (end 88.15 73.2) (width 0.7) (layer "B.Cu") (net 11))
 (segment (start 85.30016 44.92434) (end 85.30016 43.20016) (width 0.7) (layer "B.Cu") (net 11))
 (segment (start 70.67 67.07) (end 76.8 73.2) (width 0.7) (layer "B.Cu") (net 11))
 (segment (start 95.33238 80.38238) (end 95.33238 85.1182) (width 0.7) (layer "B.Cu") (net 11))
 (segment (start 88.15 73.2) (end 95.33238 80.38238) (width 0.7) (layer "B.Cu") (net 11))
 (segment (start 72.46 42.23) (end 70.67 44.02) (width 0.7) (layer "B.Cu") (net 11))
 (segment (start 84.33 42.23) (end 72.46 42.23) (width 0.7) (layer "B.Cu") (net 11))
 (segment (start 79.84 61.11) (end 81.38 62.65) (width 0.7) (layer "B.Cu") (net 8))
 (segment (start 85.30016 47.46434) (end 85.30016 50.75984) (width 0.7) (layer "B.Cu") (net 8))
 (segment (start 87.71238 61.65762) (end 87.71238 59.71566) (width 0.7) (layer "B.Cu") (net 8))
 (segment (start 83.72 52.34) (end 81.5 52.34) (width 0.7) (layer "B.Cu") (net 8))
 (segment (start 81.38 62.65) (end 86.72 62.65) (width 0.7) (layer "B.Cu") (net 8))
 (segment (start 81.5 52.34) (end 79.84 54) (width 0.7) (layer "B.Cu") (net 8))
 (segment (start 85.30016 50.75984) (end 83.72 52.34) (width 0.7) (layer "B.Cu") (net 8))
 (segment (start 86.72 62.65) (end 87.71238 61.65762) (width 0.7) (layer "B.Cu") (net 8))
 (segment (start 79.84 54) (end 79.84 61.11) (width 0.7) (layer "B.Cu") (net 8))
 (segment (start 90.25238 62.38762) (end 90.25238 59.71566) (width 0.7) (layer "B.Cu") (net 7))
 (segment (start 78.3 61.7) (end 80.9 64.3) (width 0.7) (layer "B.Cu") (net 7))
 (segment (start 80.9 64.3) (end 88.34 64.3) (width 0.7) (layer "B.Cu") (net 7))
 (segment (start 82.76016 47.46434) (end 82.76016 48.875626) (width 0.7) (layer "B.Cu") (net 7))
 (segment (start 78.3 53.335786) (end 78.3 61.7) (width 0.7) (layer "B.Cu") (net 7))
 (segment (start 82.76016 48.875626) (end 78.3 53.335786) (width 0.7) (layer "B.Cu") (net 7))
 (segment (start 88.34 64.3) (end 90.25238 62.38762) (width 0.7) (layer "B.Cu") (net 7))
 (segment (start 73.28 43.3) (end 71.95 44.63) (width 0.7) (layer "F.Cu") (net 12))
 (segment (start 79.6 43.3) (end 73.28 43.3) (width 0.7) (layer "F.Cu") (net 12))
 (segment (start 80.22016 43.92016) (end 79.6 43.3) (width 0.7) (layer "F.Cu") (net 12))
 (segment (start 90.05 74.26) (end 97.87238 82.08238) (width 0.7) (layer "F.Cu") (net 12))
 (segment (start 86.39 74.26) (end 90.05 74.26) (width 0.7) (layer "F.Cu") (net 12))
 (segment (start 80.22016 44.92434) (end 80.22016 43.92016) (width 0.7) (layer "F.Cu") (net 12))
 (segment (start 71.95 59.82) (end 86.39 74.26) (width 0.7) (layer "F.Cu") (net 12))
 (segment (start 71.95 44.63) (end 71.95 59.82) (width 0.7) (layer "F.Cu") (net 12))
 (segment (start 97.87238 82.08238) (end 97.87238 85.1182) (width 0.7) (layer "F.Cu") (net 12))
 (segment (start 76.88 43.31) (end 73.28 43.31) (width 0.7) (layer "B.Cu") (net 6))
 (segment (start 73.28 43.31) (end 71.95 44.64) (width 0.7) (layer "B.Cu") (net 6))
 (segment (start 71.95 44.64) (end 71.95 64.71) (width 0.7) (layer "B.Cu") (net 6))
 (segment (start 77.68016 44.92434) (end 77.68016 44.11016) (width 0.7) (layer "B.Cu") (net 6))
 (segment (start 100.40984 79.82984) (end 100.40984 85.1182) (width 0.7) (layer "B.Cu") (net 6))
 (segment (start 71.95 64.71) (end 78.04 70.8) (width 0.7) (layer "B.Cu") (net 6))
 (segment (start 78.04 70.8) (end 91.38 70.8) (width 0.7) (layer "B.Cu") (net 6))
 (segment (start 91.38 70.8) (end 100.40984 79.82984) (width 0.7) (layer "B.Cu") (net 6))
 (segment (start 77.68016 44.11016) (end 76.88 43.31) (width 0.7) (layer "B.Cu") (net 6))
 (segment (start 76.8 62.17) (end 76.8 51.45) (width 0.7) (layer "B.Cu") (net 9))
 (segment (start 77.68016 50.56984) (end 77.68016 47.46434) (width 0.7) (layer "B.Cu") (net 9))
 (segment (start 80.31 65.68) (end 76.8 62.17) (width 0.7) (layer "B.Cu") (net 9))
 (segment (start 92.79238 62.17762) (end 89.29 65.68) (width 0.7) (layer "B.Cu") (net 9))
 (segment (start 76.8 51.45) (end 77.68016 50.56984) (width 0.7) (layer "B.Cu") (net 9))
 (segment (start 89.29 65.68) (end 80.31 65.68) (width 0.7) (layer "B.Cu") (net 9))
 (segment (start 92.79238 59.71566) (end 92.79238 62.17762) (width 0.7) (layer "B.Cu") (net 9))
 (segment (start 78.7 68.48) (end 94.51 68.48) (width 0.7) (layer "B.Cu") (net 19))
 (segment (start 75.14016 44.92434) (end 74.13566 44.92434) (width 0.7) (layer "B.Cu") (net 19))
 (segment (start 73.22 63) (end 78.7 68.48) (width 0.7) (layer "B.Cu") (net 19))
 (segment (start 73.22 45.84) (end 73.22 63) (width 0.7) (layer "B.Cu") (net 19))
 (segment (start 97.87238 65.11762) (end 97.87238 59.71566) (width 0.7) (layer "B.Cu") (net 19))
 (segment (start 94.51 68.48) (end 97.87238 65.11762) (width 0.7) (layer "B.Cu") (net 19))
 (segment (start 74.13566 44.92434) (end 73.22 45.84) (width 0.7) (layer "B.Cu") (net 19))
 (segment (start 95.33238 63.62762) (end 95.33238 59.71566) (width 0.7) (layer "B.Cu") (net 20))
 (segment (start 79.59 67.09) (end 91.87 67.09) (width 0.7) (layer "B.Cu") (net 20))
 (segment (start 75.14016 62.64016) (end 79.59 67.09) (width 0.7) (layer "B.Cu") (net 20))
 (segment (start 91.87 67.09) (end 95.33238 63.62762) (width 0.7) (layer "B.Cu") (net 20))
 (segment (start 75.14016 47.46434) (end 75.14016 62.64016) (width 0.7) (layer "B.Cu") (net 20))
 (segment (start 110.41 53.74) (end 107.13 53.74) (width 0.7) (layer "F.Cu") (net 21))
 (segment (start 105.48984 55.38016) (end 105.48984 59.71566) (width 0.7) (layer "F.Cu") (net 21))
 (segment (start 113.24016 47.46434) (end 113.24016 50.90984) (width 0.7) (layer "F.Cu") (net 21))
 (segment (start 107.13 53.74) (end 105.48984 55.38016) (width 0.7) (layer "F.Cu") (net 21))
 (segment (start 113.24016 50.90984) (end 110.41 53.74) (width 0.7) (layer "F.Cu") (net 21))
 (segment (start 113.18 47.5245) (end 113.24016 47.46434) (width 0.7) (layer "B.Cu") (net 21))
 (segment (start 105.56 59.6455) (end 105.48984 59.71566) (width 0.7) (layer "B.Cu") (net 21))
 (segment (start 120.86016 47.46434) (end 113.24016 47.46434) (width 0.7) (layer "B.Cu") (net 21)))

